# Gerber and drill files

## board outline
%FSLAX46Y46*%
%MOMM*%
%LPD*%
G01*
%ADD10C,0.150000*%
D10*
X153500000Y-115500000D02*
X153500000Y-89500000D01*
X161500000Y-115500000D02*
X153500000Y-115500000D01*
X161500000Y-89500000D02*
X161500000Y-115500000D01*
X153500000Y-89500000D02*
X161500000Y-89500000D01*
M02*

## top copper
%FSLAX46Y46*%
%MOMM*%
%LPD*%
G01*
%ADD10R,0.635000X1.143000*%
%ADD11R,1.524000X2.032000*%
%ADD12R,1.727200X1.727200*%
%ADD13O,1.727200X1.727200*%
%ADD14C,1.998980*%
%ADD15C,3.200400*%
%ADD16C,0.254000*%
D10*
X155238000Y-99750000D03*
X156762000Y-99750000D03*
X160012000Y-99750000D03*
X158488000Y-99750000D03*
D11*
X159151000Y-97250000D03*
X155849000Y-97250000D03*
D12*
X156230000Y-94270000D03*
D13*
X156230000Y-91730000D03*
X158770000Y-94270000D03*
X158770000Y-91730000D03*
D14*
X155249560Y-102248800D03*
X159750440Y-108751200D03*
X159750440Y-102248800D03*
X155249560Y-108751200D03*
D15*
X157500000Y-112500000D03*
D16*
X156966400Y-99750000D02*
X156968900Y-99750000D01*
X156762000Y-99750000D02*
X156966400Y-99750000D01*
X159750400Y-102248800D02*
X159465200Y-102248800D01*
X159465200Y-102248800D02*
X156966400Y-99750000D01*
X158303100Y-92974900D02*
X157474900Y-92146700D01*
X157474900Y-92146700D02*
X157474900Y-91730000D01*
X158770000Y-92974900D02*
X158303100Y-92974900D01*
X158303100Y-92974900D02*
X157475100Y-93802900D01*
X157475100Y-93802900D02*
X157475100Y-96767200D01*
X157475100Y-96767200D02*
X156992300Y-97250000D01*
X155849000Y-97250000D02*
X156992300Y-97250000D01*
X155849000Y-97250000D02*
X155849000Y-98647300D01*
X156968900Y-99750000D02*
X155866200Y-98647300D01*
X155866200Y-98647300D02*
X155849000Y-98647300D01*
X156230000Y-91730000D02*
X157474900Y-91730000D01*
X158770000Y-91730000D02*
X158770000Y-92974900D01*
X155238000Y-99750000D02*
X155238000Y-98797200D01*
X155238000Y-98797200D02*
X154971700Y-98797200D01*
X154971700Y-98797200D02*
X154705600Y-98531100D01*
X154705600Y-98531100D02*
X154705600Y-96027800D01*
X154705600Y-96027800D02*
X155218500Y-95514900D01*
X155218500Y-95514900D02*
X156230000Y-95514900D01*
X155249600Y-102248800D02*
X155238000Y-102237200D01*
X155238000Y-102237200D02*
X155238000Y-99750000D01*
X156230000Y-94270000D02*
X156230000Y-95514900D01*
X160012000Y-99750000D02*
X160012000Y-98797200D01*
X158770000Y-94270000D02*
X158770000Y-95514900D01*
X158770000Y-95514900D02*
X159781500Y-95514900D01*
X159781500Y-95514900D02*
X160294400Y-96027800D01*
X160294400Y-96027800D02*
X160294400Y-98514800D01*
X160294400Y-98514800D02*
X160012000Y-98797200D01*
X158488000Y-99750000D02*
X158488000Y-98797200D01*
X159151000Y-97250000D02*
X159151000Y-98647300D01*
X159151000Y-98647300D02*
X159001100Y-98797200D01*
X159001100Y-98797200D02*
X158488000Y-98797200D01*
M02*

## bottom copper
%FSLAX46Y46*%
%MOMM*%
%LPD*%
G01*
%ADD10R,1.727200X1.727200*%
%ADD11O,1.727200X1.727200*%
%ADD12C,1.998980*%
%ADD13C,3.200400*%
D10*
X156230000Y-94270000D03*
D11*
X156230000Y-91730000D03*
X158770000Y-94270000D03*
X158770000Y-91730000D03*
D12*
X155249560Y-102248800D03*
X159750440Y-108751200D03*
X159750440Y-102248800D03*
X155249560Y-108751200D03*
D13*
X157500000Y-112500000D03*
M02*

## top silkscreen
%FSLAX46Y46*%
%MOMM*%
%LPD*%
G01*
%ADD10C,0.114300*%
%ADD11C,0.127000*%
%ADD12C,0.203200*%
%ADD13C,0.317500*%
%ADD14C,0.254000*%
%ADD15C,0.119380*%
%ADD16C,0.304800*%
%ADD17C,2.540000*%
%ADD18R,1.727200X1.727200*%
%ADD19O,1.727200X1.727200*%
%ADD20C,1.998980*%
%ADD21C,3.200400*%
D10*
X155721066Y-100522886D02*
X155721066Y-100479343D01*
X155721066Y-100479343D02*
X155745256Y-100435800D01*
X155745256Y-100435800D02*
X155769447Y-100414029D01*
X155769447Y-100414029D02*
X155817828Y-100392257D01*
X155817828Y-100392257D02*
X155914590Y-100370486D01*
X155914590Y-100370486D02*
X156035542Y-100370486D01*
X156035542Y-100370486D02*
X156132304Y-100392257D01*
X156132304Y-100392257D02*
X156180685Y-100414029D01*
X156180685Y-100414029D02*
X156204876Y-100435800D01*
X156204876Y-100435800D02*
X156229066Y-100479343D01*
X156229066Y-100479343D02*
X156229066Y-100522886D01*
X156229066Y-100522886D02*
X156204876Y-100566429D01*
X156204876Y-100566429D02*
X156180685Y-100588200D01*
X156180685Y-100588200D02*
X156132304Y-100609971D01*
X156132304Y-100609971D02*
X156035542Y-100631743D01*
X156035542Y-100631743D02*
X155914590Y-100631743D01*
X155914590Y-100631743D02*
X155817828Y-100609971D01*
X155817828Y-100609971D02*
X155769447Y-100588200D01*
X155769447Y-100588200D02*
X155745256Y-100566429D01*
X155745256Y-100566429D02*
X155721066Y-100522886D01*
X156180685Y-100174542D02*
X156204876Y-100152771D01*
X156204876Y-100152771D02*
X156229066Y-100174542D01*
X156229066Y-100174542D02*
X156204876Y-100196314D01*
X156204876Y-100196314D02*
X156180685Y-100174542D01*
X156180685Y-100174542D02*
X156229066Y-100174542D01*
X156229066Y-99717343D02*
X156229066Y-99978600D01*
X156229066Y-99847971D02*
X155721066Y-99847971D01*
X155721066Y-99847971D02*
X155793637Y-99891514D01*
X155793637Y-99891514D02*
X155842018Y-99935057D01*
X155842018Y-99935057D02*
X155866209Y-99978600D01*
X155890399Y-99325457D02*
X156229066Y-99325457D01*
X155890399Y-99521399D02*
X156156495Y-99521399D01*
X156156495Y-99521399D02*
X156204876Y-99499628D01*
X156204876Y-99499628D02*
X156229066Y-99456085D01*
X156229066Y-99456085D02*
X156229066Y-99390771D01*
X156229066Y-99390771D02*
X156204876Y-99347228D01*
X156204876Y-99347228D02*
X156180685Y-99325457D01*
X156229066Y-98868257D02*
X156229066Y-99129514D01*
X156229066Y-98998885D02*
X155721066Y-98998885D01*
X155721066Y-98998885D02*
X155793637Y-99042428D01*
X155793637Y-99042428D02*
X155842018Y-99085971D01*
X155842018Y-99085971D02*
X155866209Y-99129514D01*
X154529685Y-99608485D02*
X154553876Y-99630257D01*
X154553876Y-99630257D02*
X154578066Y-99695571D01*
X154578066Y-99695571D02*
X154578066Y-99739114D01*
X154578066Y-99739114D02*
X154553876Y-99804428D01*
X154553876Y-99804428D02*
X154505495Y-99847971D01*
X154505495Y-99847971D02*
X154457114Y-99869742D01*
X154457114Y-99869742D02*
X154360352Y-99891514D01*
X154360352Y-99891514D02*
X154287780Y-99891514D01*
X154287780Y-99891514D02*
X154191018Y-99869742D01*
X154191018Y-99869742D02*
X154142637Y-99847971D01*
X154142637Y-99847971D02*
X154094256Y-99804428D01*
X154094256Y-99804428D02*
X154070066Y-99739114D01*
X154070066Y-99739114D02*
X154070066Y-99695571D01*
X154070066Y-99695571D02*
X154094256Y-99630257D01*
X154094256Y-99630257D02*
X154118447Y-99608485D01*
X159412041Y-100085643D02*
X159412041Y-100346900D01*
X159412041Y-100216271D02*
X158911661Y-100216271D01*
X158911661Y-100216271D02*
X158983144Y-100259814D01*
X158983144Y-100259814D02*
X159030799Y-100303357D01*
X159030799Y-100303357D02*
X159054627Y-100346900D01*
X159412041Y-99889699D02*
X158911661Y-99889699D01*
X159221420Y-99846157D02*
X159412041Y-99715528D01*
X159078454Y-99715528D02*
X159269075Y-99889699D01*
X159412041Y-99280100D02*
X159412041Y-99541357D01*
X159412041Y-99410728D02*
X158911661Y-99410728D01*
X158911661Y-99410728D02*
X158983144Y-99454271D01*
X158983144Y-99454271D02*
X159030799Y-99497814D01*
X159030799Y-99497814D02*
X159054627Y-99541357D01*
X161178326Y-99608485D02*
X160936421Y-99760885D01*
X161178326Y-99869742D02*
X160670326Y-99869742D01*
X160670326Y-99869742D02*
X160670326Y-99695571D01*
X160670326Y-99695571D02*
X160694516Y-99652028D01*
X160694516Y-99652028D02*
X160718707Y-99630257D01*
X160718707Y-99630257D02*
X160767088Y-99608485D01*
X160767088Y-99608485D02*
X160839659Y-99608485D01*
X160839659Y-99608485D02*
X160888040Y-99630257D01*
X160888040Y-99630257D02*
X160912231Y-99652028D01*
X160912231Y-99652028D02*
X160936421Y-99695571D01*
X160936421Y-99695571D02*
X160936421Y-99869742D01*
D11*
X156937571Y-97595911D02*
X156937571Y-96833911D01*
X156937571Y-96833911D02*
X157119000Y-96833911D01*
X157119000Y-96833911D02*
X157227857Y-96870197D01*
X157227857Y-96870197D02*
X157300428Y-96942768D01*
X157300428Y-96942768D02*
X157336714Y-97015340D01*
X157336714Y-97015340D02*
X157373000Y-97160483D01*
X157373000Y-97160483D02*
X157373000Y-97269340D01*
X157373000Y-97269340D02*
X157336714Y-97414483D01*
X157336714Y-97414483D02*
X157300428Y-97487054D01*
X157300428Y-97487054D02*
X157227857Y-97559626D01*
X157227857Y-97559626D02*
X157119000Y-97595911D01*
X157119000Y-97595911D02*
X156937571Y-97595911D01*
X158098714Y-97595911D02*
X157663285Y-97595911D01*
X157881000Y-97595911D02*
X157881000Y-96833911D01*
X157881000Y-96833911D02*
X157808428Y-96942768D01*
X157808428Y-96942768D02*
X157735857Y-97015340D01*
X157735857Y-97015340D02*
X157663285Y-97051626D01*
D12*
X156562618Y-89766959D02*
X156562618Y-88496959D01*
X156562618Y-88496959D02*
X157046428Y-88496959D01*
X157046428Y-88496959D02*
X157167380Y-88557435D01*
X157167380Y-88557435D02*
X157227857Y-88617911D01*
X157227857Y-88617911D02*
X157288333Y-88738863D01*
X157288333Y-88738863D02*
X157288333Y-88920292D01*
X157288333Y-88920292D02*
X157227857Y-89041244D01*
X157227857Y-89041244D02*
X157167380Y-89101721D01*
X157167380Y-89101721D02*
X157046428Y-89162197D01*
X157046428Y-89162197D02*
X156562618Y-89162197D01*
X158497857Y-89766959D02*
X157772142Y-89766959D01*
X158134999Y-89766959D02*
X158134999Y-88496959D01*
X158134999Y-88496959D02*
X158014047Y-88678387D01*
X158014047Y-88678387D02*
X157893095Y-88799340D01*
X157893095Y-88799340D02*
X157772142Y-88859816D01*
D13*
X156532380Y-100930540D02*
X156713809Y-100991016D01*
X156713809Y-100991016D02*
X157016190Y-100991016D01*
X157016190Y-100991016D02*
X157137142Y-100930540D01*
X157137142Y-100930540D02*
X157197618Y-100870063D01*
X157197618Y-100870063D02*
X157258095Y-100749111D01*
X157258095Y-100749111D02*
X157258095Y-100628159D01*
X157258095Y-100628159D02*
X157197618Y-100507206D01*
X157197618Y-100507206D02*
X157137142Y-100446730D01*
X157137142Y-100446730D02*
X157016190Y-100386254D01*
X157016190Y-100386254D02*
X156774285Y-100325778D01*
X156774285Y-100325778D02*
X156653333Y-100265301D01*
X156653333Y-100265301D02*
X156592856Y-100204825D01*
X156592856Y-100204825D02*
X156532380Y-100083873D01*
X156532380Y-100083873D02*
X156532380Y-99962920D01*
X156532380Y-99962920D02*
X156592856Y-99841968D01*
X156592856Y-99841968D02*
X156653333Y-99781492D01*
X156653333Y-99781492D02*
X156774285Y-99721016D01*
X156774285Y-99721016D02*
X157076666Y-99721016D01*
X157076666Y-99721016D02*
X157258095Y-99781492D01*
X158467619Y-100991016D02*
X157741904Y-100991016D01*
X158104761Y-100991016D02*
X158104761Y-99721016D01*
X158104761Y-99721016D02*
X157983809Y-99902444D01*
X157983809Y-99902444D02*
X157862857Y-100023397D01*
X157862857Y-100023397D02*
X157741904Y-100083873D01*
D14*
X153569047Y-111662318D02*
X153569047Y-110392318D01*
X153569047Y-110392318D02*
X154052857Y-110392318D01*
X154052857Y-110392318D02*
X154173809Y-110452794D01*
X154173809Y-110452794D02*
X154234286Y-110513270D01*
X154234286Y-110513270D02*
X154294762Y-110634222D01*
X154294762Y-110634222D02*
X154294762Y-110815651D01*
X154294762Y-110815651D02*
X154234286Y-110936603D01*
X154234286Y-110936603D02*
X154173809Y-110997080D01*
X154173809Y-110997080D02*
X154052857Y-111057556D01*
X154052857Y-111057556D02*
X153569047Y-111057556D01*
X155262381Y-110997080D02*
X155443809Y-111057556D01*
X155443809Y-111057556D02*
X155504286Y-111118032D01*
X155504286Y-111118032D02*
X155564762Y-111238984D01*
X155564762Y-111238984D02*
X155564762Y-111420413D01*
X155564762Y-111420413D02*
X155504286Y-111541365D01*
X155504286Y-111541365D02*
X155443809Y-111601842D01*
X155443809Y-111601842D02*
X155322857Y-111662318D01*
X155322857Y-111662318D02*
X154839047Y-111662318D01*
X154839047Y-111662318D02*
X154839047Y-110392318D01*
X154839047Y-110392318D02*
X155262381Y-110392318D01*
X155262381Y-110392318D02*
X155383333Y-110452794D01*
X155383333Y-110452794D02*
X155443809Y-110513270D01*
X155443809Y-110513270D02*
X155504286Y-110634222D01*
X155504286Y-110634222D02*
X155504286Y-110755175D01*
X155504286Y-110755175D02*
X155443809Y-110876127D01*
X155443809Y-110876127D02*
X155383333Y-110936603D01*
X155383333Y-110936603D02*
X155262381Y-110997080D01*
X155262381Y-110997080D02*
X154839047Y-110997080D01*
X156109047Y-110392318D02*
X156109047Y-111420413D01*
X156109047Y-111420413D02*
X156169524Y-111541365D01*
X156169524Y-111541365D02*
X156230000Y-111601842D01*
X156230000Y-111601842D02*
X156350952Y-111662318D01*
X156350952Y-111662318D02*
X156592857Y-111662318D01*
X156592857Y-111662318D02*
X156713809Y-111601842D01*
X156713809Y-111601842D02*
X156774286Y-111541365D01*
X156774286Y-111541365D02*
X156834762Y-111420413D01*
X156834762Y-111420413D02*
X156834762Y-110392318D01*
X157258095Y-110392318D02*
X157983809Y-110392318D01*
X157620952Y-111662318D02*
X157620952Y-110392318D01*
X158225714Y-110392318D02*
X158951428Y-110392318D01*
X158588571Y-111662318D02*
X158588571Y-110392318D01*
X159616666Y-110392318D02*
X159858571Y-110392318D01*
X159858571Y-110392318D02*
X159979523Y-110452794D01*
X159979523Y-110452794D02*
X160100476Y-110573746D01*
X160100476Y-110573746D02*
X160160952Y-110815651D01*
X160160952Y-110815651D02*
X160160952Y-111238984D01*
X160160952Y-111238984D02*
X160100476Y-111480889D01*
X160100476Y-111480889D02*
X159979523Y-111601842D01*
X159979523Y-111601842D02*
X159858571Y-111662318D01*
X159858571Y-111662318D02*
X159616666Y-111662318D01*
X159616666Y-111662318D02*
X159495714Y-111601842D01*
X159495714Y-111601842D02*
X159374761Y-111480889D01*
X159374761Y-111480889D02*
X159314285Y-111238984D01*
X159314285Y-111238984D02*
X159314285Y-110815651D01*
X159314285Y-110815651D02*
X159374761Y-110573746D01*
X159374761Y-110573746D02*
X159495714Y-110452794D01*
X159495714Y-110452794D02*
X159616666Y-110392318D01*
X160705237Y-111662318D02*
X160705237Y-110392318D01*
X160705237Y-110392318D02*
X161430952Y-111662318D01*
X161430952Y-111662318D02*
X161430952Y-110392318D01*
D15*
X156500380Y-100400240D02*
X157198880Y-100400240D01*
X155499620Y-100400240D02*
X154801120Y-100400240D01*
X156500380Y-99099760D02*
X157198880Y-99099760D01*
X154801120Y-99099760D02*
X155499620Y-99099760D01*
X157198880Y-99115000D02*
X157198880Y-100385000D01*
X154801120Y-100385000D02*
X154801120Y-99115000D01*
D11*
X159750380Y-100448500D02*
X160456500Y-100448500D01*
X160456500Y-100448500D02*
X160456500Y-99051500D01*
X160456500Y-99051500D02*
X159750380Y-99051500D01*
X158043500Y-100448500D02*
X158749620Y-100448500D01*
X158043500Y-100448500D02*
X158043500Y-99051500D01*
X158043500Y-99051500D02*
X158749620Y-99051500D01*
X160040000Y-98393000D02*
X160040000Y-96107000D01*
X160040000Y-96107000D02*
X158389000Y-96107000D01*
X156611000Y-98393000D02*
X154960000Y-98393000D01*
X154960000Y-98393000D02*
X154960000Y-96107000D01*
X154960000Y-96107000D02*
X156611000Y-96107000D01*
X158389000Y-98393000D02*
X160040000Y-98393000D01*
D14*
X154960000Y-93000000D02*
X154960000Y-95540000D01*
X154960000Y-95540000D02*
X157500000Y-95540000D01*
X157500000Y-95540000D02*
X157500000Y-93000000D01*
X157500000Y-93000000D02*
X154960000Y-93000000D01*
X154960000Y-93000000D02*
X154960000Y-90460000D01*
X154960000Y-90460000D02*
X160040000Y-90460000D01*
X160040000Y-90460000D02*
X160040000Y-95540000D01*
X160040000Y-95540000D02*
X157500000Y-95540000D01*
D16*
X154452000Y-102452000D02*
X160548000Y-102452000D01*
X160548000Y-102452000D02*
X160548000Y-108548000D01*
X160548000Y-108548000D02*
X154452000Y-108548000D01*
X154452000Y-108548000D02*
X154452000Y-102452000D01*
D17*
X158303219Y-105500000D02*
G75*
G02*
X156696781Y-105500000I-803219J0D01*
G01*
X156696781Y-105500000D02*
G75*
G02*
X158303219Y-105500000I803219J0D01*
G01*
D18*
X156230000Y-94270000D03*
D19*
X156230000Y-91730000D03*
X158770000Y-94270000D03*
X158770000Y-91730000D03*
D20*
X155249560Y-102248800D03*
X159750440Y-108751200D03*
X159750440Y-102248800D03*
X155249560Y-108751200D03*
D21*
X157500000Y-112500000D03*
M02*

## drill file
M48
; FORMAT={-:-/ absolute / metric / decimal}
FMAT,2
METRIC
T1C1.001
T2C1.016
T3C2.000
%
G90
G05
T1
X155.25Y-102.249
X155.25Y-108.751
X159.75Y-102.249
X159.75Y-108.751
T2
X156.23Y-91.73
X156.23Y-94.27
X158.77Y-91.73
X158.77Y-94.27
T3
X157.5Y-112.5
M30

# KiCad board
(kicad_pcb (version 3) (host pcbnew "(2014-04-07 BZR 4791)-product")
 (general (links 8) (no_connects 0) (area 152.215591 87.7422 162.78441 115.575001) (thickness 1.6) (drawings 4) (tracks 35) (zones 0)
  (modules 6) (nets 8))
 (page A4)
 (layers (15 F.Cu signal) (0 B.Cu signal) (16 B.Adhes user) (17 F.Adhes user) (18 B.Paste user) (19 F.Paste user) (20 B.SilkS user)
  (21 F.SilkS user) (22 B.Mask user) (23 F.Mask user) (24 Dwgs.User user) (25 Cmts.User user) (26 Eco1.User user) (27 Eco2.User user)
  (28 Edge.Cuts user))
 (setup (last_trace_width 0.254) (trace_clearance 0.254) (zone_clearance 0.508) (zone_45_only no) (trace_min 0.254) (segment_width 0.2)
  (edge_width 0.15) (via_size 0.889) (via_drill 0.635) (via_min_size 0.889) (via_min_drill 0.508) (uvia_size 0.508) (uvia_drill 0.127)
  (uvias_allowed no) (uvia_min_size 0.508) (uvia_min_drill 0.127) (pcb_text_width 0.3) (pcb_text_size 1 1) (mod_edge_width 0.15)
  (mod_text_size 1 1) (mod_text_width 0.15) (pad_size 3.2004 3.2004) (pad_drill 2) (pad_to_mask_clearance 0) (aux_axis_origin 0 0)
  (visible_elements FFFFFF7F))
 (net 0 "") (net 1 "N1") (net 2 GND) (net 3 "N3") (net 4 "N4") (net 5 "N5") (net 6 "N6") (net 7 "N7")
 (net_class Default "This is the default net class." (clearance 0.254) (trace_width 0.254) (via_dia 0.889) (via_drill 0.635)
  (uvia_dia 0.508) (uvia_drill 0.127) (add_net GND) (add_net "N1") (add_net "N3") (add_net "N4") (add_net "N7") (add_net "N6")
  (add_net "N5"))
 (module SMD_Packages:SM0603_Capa (layer F.Cu) (at 156 99.75)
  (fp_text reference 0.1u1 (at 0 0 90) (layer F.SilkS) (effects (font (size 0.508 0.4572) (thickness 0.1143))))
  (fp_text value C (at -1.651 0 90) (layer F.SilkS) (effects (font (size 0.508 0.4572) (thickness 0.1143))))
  (fp_line (start 0.50038 0.65024) (end 1.19888 0.65024) (layer F.SilkS) (width 0.11938))
  (fp_line (start -0.50038 0.65024) (end -1.19888 0.65024) (layer F.SilkS) (width 0.11938))
  (fp_line (start 0.50038 -0.65024) (end 1.19888 -0.65024) (layer F.SilkS) (width 0.11938))
  (fp_line (start -1.19888 -0.65024) (end -0.50038 -0.65024) (layer F.SilkS) (width 0.11938))
  (fp_line (start 1.19888 -0.635) (end 1.19888 0.635) (layer F.SilkS) (width 0.11938))
  (fp_line (start -1.19888 0.635) (end -1.19888 -0.635) (layer F.SilkS) (width 0.11938))
  (pad 1 smd rect (at -0.762 0) (size 0.635 1.143) (layers F.Cu F.Paste F.Mask) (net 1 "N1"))
  (pad 2 smd rect (at 0.762 0) (size 0.635 1.143) (layers F.Cu F.Paste F.Mask) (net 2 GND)))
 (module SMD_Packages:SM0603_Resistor (layer F.Cu) (at 159.25 99.75 180)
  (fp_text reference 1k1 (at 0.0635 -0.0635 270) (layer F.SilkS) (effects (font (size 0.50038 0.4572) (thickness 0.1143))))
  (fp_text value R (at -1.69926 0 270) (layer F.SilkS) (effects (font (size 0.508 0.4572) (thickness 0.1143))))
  (fp_line (start -0.50038 -0.6985) (end -1.2065 -0.6985) (layer F.SilkS) (width 0.127))
  (fp_line (start -1.2065 -0.6985) (end -1.2065 0.6985) (layer F.SilkS) (width 0.127))
  (fp_line (start -1.2065 0.6985) (end -0.50038 0.6985) (layer F.SilkS) (width 0.127))
  (fp_line (start 1.2065 -0.6985) (end 0.50038 -0.6985) (layer F.SilkS) (width 0.127))
  (fp_line (start 1.2065 -0.6985) (end 1.2065 0.6985) (layer F.SilkS) (width 0.127))
  (fp_line (start 1.2065 0.6985) (end 0.50038 0.6985) (layer F.SilkS) (width 0.127))
  (pad 1 smd rect (at -0.762 0 180) (size 0.635 1.143) (layers F.Cu F.Paste F.Mask) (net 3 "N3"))
  (pad 2 smd rect (at 0.762 0 180) (size 0.635 1.143) (layers F.Cu F.Paste F.Mask) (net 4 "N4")))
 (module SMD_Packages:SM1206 (layer F.Cu) (at 157.5 97.25 180)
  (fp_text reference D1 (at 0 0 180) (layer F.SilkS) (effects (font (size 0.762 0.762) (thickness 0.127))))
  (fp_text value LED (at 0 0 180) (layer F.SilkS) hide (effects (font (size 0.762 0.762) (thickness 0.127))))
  (fp_line (start -2.54 -1.143) (end -2.54 1.143) (layer F.SilkS) (width 0.127))
  (fp_line (start -2.54 1.143) (end -0.889 1.143) (layer F.SilkS) (width 0.127))
  (fp_line (start 0.889 -1.143) (end 2.54 -1.143) (layer F.SilkS) (width 0.127))
  (fp_line (start 2.54 -1.143) (end 2.54 1.143) (layer F.SilkS) (width 0.127))
  (fp_line (start 2.54 1.143) (end 0.889 1.143) (layer F.SilkS) (width 0.127))
  (fp_line (start -0.889 -1.143) (end -2.54 -1.143) (layer F.SilkS) (width 0.127))
  (pad 1 smd rect (at -1.651 0 180) (size 1.524 2.032) (layers F.Cu F.Paste F.Mask) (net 4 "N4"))
  (pad 2 smd rect (at 1.651 0 180) (size 1.524 2.032) (layers F.Cu F.Paste F.Mask) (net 2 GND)))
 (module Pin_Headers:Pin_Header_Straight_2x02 (layer F.Cu) (at 157.5 93)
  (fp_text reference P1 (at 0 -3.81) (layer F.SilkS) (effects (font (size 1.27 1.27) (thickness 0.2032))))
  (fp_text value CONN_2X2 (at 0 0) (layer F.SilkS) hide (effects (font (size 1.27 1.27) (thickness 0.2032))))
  (fp_line (start -2.54 0) (end -2.54 2.54) (layer F.SilkS) (width 0.254))
  (fp_line (start -2.54 2.54) (end 0 2.54) (layer F.SilkS) (width 0.254))
  (fp_line (start 0 2.54) (end 0 0) (layer F.SilkS) (width 0.254))
  (fp_line (start 0 0) (end -2.54 0) (layer F.SilkS) (width 0.254))
  (fp_line (start -2.54 0) (end -2.54 -2.54) (layer F.SilkS) (width 0.254))
  (fp_line (start -2.54 -2.54) (end 2.54 -2.54) (layer F.SilkS) (width 0.254))
  (fp_line (start 2.54 -2.54) (end 2.54 2.54) (layer F.SilkS) (width 0.254))
  (fp_line (start 2.54 2.54) (end 0 2.54) (layer F.SilkS) (width 0.254))
  (pad 1 thru_hole rect (at -1.27 1.27) (size 1.7272 1.7272) (drill 1.016) (layers *.Cu *.Mask F.SilkS) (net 1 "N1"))
  (pad 2 thru_hole oval (at -1.27 -1.27) (size 1.7272 1.7272) (drill 1.016) (layers *.Cu *.Mask F.SilkS) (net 2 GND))
  (pad 3 thru_hole oval (at 1.27 1.27) (size 1.7272 1.7272) (drill 1.016) (layers *.Cu *.Mask F.SilkS) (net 3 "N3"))
  (pad 4 thru_hole oval (at 1.27 -1.27) (size 1.7272 1.7272) (drill 1.016) (layers *.Cu *.Mask F.SilkS) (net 2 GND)))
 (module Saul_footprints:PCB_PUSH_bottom (layer F.Cu) (at 157.5 105.5)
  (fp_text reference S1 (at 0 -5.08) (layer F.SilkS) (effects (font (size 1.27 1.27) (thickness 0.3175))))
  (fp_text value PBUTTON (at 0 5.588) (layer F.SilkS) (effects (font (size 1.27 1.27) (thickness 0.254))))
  (fp_line (start -3.048 -3.048) (end 3.048 -3.048) (layer F.SilkS) (width 0.3048))
  (fp_line (start 3.048 -3.048) (end 3.048 3.048) (layer F.SilkS) (width 0.3048))
  (fp_line (start 3.048 3.048) (end -3.048 3.048) (layer F.SilkS) (width 0.3048))
  (fp_line (start -3.048 3.048) (end -3.048 -3.048) (layer F.SilkS) (width 0.3048))
  (fp_circle (center 0 0) (end -0.762 0.254) (layer F.SilkS) (width 2.54))
  (pad 1 thru_hole circle (at -2.25044 -3.2512) (size 1.99898 1.99898) (drill 1.00076) (layers *.Cu *.Mask F.SilkS) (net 1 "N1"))
  (pad 3 thru_hole circle (at 2.25044 3.2512) (size 1.99898 1.99898) (drill 1.00076) (layers *.Cu *.Mask F.SilkS) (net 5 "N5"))
  (pad 4 thru_hole circle (at 2.25044 -3.2512) (size 1.99898 1.99898) (drill 1.00076) (layers *.Cu *.Mask F.SilkS) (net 2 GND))
  (pad 2 thru_hole circle (at -2.25044 3.2512) (size 1.99898 1.99898) (drill 1.00076) (layers *.Cu *.Mask F.SilkS) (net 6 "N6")))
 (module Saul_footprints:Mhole (layer F.Cu) (at 157.5 112.5)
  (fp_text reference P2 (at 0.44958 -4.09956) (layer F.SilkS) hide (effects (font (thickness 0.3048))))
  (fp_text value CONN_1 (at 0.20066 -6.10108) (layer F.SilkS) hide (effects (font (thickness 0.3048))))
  (pad 1 thru_hole circle (at 0 0) (size 3.2004 3.2004) (drill 2) (layers *.Cu *.Mask F.SilkS) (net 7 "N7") (clearance 1.00076)))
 (gr_line (start 153.5 115.5) (end 153.5 89.5) (angle 90) (layer Edge.Cuts) (width 0.15))
 (gr_line (start 161.5 115.5) (end 153.5 115.5) (angle 90) (layer Edge.Cuts) (width 0.15))
 (gr_line (start 161.5 89.5) (end 161.5 115.5) (angle 90) (layer Edge.Cuts) (width 0.15))
 (gr_line (start 153.5 89.5) (end 161.5 89.5) (angle 90) (layer Edge.Cuts) (width 0.15))
 (segment (start 156.9664 99.75) (end 156.9689 99.75) (width 0.254) (layer F.Cu) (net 2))
 (segment (start 156.762 99.75) (end 156.9664 99.75) (width 0.254) (layer F.Cu) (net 2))
 (segment (start 159.7504 102.2488) (end 159.4652 102.2488) (width 0.254) (layer F.Cu) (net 2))
 (segment (start 159.4652 102.2488) (end 156.9664 99.75) (width 0.254) (layer F.Cu) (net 2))
 (segment (start 158.3031 92.9749) (end 157.4749 92.1467) (width 0.254) (layer F.Cu) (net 2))
 (segment (start 157.4749 92.1467) (end 157.4749 91.73) (width 0.254) (layer F.Cu) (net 2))
 (segment (start 158.77 92.9749) (end 158.3031 92.9749) (width 0.254) (layer F.Cu) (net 2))
 (segment (start 158.3031 92.9749) (end 157.4751 93.8029) (width 0.254) (layer F.Cu) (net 2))
 (segment (start 157.4751 93.8029) (end 157.4751 96.7672) (width 0.254) (layer F.Cu) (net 2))
 (segment (start 157.4751 96.7672) (end 156.9923 97.25) (width 0.254) (layer F.Cu) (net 2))
 (segment (start 155.849 97.25) (end 156.9923 97.25) (width 0.254) (layer F.Cu) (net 2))
 (segment (start 155.849 97.25) (end 155.849 98.6473) (width 0.254) (layer F.Cu) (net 2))
 (segment (start 156.9689 99.75) (end 155.8662 98.6473) (width 0.254) (layer F.Cu) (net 2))
 (segment (start 155.8662 98.6473) (end 155.849 98.6473) (width 0.254) (layer F.Cu) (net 2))
 (segment (start 156.23 91.73) (end 157.4749 91.73) (width 0.254) (layer F.Cu) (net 2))
 (segment (start 158.77 91.73) (end 158.77 92.9749) (width 0.254) (layer F.Cu) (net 2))
 (segment (start 155.238 99.75) (end 155.238 98.7972) (width 0.254) (layer F.Cu) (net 1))
 (segment (start 155.238 98.7972) (end 154.9717 98.7972) (width 0.254) (layer F.Cu) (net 1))
 (segment (start 154.9717 98.7972) (end 154.7056 98.5311) (width 0.254) (layer F.Cu) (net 1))
 (segment (start 154.7056 98.5311) (end 154.7056 96.0278) (width 0.254) (layer F.Cu) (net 1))
 (segment (start 154.7056 96.0278) (end 155.2185 95.5149) (width 0.254) (layer F.Cu) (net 1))
 (segment (start 155.2185 95.5149) (end 156.23 95.5149) (width 0.254) (layer F.Cu) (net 1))
 (segment (start 155.2496 102.2488) (end 155.238 102.2372) (width 0.254) (layer F.Cu) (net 1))
 (segment (start 155.238 102.2372) (end 155.238 99.75) (width 0.254) (layer F.Cu) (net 1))
 (segment (start 156.23 94.27) (end 156.23 95.5149) (width 0.254) (layer F.Cu) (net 1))
 (segment (start 160.012 99.75) (end 160.012 98.7972) (width 0.254) (layer F.Cu) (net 3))
 (segment (start 158.77 94.27) (end 158.77 95.5149) (width 0.254) (layer F.Cu) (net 3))
 (segment (start 158.77 95.5149) (end 159.7815 95.5149) (width 0.254) (layer F.Cu) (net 3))
 (segment (start 159.7815 95.5149) (end 160.2944 96.0278) (width 0.254) (layer F.Cu) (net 3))
 (segment (start 160.2944 96.0278) (end 160.2944 98.5148) (width 0.254) (layer F.Cu) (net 3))
 (segment (start 160.2944 98.5148) (end 160.012 98.7972) (width 0.254) (layer F.Cu) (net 3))
 (segment (start 158.488 99.75) (end 158.488 98.7972) (width 0.254) (layer F.Cu) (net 4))
 (segment (start 159.151 97.25) (end 159.151 98.6473) (width 0.254) (layer F.Cu) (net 4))
 (segment (start 159.151 98.6473) (end 159.0011 98.7972) (width 0.254) (layer F.Cu) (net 4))
 (segment (start 159.0011 98.7972) (end 158.488 98.7972) (width 0.254) (layer F.Cu) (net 4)))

